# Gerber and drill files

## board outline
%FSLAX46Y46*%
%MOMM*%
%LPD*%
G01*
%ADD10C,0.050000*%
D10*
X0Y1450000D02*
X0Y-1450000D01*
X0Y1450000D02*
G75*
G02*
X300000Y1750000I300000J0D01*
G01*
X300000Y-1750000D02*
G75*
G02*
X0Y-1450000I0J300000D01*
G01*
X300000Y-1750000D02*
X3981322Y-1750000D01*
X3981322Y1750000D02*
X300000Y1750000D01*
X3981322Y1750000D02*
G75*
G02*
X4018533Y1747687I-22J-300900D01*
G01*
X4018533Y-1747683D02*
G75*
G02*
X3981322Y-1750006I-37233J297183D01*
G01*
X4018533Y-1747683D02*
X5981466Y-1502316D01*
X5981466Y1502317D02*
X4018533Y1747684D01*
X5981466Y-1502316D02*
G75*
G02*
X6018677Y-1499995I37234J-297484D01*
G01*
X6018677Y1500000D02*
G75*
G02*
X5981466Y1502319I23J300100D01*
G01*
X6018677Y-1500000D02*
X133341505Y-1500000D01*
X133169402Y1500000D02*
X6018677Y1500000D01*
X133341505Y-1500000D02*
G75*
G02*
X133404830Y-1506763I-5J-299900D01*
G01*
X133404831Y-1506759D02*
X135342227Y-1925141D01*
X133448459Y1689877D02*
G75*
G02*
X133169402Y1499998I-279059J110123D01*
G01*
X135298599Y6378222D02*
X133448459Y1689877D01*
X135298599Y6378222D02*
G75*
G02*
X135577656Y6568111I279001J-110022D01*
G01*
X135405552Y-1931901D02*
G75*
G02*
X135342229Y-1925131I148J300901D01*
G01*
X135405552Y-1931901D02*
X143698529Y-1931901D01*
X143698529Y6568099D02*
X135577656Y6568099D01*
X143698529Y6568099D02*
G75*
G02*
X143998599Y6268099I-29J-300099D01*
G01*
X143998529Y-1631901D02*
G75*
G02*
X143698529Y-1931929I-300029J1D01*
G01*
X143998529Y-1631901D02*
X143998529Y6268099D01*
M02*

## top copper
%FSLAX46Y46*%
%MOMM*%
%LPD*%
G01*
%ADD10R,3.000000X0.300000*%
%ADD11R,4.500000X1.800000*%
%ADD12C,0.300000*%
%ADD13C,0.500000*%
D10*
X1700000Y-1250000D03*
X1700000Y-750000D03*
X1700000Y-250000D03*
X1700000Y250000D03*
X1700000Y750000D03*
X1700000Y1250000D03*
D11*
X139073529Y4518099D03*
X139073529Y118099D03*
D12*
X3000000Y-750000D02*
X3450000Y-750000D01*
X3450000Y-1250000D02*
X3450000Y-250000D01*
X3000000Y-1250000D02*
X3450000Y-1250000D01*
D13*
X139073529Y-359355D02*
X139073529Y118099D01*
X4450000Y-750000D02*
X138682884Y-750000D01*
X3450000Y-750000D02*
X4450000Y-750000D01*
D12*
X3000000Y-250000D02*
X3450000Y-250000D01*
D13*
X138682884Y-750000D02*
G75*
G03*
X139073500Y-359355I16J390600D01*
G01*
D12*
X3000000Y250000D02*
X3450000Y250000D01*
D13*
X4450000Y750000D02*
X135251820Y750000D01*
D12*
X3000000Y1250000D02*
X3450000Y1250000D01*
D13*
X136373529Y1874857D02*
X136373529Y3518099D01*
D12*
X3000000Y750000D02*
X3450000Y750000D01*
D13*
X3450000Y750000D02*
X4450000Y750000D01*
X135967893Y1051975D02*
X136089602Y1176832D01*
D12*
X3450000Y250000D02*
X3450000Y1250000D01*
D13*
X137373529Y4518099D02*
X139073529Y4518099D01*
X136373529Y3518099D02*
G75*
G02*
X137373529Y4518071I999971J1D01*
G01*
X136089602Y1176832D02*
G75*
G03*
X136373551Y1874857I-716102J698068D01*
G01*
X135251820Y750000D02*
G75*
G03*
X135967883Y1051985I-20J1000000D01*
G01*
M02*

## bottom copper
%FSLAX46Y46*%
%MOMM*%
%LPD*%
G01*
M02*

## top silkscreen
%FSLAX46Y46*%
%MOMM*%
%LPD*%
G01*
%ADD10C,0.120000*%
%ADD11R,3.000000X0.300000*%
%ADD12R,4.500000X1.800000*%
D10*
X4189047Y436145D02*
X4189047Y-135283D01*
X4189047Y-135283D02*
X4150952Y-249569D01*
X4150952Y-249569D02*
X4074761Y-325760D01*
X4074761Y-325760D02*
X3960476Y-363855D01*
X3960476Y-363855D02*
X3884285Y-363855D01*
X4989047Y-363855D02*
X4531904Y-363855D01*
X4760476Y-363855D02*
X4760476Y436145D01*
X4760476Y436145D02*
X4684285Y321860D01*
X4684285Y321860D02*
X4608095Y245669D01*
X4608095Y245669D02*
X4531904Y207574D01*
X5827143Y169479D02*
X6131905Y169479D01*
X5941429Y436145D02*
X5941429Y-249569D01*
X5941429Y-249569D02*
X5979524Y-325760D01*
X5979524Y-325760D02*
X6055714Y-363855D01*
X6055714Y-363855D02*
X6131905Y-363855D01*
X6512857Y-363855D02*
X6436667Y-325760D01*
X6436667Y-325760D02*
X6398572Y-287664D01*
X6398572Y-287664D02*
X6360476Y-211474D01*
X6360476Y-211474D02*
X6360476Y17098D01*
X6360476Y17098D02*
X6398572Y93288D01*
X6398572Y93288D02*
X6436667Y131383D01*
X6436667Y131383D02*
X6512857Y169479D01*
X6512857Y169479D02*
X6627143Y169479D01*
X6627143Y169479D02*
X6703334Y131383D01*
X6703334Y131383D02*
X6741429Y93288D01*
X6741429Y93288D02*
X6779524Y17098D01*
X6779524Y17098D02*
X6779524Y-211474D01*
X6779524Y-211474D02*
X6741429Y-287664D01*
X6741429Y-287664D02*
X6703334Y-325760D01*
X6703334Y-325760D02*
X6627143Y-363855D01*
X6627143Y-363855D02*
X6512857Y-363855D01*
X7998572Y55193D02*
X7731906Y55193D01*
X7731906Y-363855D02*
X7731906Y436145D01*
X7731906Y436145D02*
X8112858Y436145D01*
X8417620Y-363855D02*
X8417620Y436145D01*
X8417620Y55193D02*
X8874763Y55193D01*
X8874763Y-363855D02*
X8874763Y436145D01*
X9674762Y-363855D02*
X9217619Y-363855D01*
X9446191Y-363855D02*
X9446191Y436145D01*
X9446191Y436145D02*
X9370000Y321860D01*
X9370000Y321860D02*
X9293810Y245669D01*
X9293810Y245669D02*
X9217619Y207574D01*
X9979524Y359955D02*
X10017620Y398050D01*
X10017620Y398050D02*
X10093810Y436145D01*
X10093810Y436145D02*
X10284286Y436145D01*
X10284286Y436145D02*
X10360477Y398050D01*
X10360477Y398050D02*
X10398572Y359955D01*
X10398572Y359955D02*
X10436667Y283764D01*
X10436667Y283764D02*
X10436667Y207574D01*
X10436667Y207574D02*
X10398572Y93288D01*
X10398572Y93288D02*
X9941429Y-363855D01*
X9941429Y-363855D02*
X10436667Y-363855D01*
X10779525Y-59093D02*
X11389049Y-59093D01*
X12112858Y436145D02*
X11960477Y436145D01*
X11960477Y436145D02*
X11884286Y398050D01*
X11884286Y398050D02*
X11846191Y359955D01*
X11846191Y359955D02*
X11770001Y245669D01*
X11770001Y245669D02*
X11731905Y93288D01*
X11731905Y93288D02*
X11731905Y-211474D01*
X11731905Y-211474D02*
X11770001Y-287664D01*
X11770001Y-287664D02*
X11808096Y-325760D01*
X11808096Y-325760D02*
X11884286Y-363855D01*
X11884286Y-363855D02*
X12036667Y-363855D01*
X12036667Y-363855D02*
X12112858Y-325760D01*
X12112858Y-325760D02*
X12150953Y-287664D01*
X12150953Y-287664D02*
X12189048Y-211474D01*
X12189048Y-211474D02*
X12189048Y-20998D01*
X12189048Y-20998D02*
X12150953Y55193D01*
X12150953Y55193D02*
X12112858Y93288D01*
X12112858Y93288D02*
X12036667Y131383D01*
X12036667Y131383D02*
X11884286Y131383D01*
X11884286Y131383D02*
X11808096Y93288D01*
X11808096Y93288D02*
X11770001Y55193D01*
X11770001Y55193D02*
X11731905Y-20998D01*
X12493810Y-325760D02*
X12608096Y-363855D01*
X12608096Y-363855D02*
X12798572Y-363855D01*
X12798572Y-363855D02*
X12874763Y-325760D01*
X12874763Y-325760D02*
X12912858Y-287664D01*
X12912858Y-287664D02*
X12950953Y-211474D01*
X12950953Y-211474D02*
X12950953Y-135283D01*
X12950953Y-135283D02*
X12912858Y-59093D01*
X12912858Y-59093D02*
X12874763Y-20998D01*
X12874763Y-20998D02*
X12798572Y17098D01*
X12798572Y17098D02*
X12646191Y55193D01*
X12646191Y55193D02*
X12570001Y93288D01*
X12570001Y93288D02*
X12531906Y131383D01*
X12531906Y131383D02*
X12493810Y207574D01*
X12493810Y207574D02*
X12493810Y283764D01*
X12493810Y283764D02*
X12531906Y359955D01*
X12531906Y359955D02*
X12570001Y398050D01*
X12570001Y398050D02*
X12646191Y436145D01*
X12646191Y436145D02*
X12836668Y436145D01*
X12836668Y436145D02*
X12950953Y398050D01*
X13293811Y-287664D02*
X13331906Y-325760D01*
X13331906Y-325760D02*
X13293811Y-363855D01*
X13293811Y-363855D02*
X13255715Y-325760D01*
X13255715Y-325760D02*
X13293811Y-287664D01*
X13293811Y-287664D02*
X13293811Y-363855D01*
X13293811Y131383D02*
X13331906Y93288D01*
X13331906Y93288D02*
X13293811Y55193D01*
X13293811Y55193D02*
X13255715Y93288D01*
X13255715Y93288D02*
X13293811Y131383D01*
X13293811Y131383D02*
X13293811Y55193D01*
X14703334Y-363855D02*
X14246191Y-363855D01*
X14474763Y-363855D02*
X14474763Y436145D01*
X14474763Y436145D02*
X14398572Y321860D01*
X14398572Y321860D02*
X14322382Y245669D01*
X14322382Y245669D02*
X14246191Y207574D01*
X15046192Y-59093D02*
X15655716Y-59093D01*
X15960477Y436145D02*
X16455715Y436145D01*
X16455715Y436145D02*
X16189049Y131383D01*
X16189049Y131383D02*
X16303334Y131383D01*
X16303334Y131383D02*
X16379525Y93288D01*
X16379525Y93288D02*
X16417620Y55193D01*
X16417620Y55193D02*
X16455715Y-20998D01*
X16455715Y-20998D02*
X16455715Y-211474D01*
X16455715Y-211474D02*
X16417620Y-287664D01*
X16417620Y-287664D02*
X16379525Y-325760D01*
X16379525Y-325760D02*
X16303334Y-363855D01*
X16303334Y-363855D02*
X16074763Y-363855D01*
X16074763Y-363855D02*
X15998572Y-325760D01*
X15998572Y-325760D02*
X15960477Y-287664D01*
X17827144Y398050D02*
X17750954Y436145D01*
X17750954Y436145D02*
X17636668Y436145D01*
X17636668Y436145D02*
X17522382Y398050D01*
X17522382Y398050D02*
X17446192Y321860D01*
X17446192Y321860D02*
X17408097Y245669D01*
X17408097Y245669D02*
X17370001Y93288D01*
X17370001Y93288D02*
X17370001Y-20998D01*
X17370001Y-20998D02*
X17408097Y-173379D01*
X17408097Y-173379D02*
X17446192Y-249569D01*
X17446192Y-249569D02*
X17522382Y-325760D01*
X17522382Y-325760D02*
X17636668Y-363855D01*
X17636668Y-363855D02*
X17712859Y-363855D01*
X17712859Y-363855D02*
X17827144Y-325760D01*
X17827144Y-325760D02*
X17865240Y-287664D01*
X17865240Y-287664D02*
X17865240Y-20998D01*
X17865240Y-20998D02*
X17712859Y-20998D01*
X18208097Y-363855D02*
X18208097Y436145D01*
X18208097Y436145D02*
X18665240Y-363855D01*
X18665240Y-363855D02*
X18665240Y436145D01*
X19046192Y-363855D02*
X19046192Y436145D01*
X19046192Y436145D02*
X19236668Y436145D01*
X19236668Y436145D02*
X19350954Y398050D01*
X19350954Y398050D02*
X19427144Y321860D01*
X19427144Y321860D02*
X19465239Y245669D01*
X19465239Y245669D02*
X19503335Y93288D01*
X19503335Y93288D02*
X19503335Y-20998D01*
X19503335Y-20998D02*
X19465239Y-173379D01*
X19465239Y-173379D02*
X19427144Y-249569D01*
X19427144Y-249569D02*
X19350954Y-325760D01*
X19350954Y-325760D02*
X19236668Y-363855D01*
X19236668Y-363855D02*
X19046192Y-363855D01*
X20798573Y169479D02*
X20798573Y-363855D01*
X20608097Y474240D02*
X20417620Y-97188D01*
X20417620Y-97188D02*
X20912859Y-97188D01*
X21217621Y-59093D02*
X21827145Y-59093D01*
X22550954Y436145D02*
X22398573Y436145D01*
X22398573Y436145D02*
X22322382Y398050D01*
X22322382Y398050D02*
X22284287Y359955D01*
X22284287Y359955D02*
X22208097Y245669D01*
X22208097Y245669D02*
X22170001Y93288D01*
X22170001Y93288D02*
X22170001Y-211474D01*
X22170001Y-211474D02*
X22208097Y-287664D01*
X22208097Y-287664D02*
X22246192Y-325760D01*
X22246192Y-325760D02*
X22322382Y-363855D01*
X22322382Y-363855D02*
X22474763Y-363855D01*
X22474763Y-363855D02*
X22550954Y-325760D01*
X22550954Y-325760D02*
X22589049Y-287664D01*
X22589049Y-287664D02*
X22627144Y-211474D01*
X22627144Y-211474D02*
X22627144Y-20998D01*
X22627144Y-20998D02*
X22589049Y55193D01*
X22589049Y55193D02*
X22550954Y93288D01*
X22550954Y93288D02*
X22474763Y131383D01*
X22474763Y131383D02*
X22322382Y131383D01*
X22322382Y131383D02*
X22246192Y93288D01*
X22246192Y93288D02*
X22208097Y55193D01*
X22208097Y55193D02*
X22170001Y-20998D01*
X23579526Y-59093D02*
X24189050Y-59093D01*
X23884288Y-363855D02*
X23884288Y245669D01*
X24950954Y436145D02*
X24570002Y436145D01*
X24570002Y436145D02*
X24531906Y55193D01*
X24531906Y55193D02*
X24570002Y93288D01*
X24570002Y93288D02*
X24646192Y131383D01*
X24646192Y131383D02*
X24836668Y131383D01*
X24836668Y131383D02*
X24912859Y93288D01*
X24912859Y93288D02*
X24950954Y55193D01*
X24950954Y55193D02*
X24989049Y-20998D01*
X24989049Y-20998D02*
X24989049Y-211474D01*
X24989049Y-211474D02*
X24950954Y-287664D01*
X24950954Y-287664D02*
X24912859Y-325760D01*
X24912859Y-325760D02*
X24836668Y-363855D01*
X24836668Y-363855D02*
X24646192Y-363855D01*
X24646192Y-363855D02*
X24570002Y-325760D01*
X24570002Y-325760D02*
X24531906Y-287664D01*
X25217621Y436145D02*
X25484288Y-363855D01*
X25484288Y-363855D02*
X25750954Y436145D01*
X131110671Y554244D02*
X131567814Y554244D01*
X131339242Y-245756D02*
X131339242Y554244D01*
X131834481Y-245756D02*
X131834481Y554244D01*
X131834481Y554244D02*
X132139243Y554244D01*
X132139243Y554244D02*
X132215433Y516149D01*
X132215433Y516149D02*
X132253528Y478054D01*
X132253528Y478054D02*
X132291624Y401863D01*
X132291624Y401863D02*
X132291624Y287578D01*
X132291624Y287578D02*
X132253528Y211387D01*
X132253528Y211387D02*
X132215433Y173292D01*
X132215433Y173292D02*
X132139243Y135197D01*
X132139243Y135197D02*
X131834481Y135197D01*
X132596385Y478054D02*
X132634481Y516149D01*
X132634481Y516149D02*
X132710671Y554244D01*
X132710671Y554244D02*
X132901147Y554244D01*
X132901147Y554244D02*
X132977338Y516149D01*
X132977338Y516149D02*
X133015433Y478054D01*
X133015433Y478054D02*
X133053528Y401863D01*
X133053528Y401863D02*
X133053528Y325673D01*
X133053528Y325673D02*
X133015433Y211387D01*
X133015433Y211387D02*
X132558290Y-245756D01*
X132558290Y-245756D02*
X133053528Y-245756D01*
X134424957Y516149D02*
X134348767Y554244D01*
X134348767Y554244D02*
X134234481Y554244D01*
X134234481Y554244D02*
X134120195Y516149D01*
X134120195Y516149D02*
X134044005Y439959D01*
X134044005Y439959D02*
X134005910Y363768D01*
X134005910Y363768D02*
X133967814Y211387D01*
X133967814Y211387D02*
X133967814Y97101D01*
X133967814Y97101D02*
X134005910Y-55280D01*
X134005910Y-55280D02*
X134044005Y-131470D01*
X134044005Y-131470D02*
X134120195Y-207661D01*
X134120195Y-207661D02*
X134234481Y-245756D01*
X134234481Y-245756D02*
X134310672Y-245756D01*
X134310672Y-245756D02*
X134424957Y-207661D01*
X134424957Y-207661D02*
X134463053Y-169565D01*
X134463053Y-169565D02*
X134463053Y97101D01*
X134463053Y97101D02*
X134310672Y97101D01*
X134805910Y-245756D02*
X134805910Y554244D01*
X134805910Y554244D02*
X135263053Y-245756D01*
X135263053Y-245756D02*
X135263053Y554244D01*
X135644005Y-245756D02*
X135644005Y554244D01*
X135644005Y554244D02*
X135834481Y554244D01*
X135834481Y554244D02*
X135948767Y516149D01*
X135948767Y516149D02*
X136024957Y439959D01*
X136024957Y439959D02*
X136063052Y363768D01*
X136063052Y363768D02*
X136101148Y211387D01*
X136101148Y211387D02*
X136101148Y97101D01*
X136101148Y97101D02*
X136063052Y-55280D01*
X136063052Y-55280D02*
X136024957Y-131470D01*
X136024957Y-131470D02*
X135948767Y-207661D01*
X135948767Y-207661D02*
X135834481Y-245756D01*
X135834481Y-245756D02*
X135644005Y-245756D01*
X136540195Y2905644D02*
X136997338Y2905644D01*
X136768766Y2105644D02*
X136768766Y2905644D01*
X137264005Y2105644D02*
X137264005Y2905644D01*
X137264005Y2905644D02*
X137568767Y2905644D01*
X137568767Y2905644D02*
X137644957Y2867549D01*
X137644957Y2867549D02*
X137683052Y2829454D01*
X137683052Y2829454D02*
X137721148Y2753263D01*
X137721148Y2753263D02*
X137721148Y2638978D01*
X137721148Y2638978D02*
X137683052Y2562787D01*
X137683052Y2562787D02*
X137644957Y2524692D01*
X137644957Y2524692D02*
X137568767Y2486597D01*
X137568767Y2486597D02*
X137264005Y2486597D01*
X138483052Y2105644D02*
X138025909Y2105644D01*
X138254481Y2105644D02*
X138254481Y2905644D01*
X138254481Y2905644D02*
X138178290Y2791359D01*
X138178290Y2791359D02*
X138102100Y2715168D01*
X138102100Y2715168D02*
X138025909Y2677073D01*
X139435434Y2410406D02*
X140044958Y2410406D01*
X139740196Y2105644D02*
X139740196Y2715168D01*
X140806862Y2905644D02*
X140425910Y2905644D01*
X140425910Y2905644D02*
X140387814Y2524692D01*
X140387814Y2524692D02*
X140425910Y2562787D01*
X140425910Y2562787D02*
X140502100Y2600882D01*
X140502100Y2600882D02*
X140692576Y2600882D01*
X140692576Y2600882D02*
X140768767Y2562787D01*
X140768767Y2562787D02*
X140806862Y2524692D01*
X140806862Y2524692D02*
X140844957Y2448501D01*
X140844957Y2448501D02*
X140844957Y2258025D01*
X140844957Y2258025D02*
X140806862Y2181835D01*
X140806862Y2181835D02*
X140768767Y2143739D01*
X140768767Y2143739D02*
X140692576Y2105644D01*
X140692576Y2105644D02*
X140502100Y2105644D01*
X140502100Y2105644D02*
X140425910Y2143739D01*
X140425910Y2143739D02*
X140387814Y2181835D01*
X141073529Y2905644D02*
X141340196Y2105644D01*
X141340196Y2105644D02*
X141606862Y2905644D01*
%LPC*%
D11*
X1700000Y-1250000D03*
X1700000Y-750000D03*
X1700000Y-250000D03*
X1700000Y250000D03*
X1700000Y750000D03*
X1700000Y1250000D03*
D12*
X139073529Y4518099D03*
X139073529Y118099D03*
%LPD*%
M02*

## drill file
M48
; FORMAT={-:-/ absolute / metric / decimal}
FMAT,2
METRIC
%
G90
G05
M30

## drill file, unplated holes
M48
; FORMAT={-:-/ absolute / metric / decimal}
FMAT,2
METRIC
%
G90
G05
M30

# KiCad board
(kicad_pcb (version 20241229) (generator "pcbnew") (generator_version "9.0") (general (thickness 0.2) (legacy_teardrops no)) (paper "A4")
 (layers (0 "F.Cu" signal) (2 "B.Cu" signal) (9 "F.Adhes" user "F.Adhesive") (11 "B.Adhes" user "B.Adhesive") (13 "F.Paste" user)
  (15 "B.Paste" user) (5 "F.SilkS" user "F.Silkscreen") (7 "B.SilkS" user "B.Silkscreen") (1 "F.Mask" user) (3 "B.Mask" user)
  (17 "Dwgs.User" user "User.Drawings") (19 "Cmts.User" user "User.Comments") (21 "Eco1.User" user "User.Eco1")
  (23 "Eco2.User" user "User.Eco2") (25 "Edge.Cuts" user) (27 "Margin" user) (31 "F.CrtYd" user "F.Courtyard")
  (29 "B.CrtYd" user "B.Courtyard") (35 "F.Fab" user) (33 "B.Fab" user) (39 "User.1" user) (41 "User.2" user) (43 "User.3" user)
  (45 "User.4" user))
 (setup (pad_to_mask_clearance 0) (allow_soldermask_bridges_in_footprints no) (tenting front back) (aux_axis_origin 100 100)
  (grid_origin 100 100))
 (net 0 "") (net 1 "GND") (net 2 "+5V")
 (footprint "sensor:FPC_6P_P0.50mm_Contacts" (layer "F.Cu") (at 101.7 100)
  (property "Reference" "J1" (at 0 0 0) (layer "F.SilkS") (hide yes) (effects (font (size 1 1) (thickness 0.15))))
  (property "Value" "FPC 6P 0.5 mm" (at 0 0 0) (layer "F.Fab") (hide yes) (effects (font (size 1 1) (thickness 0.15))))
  (pad "1" smd rect (at 0 1.25) (size 3 0.3) (layers "F.Cu" "F.Mask") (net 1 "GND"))
  (pad "2" smd rect (at 0 0.75) (size 3 0.3) (layers "F.Cu" "F.Mask") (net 1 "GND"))
  (pad "3" smd rect (at 0 0.25) (size 3 0.3) (layers "F.Cu" "F.Mask") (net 1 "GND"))
  (pad "4" smd rect (at 0 -0.25) (size 3 0.3) (layers "F.Cu" "F.Mask") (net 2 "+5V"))
  (pad "5" smd rect (at 0 -0.75) (size 3 0.3) (layers "F.Cu" "F.Mask") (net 2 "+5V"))
  (pad "6" smd rect (at 0 -1.25) (size 3 0.3) (layers "F.Cu" "F.Mask") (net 2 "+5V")))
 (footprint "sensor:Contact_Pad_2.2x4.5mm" (layer "F.Cu") (at 239.073529 95.481901)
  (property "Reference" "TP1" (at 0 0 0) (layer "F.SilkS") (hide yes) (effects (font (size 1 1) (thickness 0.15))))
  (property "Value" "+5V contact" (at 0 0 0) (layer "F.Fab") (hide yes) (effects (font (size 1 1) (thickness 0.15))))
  (pad "1" smd rect (at 0 0) (size 4.5 1.8) (layers "F.Cu" "F.Mask") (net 2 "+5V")))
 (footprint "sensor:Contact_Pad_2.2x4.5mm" (layer "F.Cu") (at 239.073529 99.881901)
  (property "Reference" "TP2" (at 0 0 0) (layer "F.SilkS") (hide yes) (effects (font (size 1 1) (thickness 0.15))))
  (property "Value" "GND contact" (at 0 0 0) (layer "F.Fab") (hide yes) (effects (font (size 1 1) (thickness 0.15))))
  (pad "1" smd rect (at 0 0) (size 4.5 1.8) (layers "F.Cu" "F.Mask") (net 1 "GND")))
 (gr_line (start 100 98.55) (end 100 101.45) (stroke (width 0.05) (type default)) (layer "Edge.Cuts"))
 (gr_arc (start 100 98.55) (mid 100.087868 98.337868) (end 100.3 98.25) (stroke (width 0.05) (type default)) (layer "Edge.Cuts"))
 (gr_arc (start 100.3 101.75) (mid 100.087868 101.662132) (end 100 101.45) (stroke (width 0.05) (type default)) (layer "Edge.Cuts"))
 (gr_line (start 100.3 101.75) (end 103.981322 101.75) (stroke (width 0.05) (type default)) (layer "Edge.Cuts"))
 (gr_line (start 103.981322 98.25) (end 100.3 98.25) (stroke (width 0.05) (type default)) (layer "Edge.Cuts"))
 (gr_arc (start 103.981322 98.25) (mid 103.999963 98.250581) (end 104.018533 98.252316) (stroke (width 0.05) (type default))
  (layer "Edge.Cuts"))
 (gr_arc (start 104.018533 101.747683) (mid 103.999964 101.749421) (end 103.981322 101.75) (stroke (width 0.05) (type default))
  (layer "Edge.Cuts"))
 (gr_line (start 104.018533 101.747683) (end 105.981466 101.502316) (stroke (width 0.05) (type default)) (layer "Edge.Cuts"))
 (gr_line (start 105.981466 98.497683) (end 104.018533 98.252316) (stroke (width 0.05) (type default)) (layer "Edge.Cuts"))
 (gr_arc (start 105.981466 101.502316) (mid 106.000036 101.500579) (end 106.018677 101.5) (stroke (width 0.05) (type default))
  (layer "Edge.Cuts"))
 (gr_arc (start 106.018677 98.5) (mid 106.000036 98.49942) (end 105.981466 98.497683) (stroke (width 0.05) (type default))
  (layer "Edge.Cuts"))
 (gr_line (start 106.018677 101.5) (end 233.341505 101.5) (stroke (width 0.05) (type default)) (layer "Edge.Cuts"))
 (gr_line (start 233.169402 98.5) (end 106.018677 98.5) (stroke (width 0.05) (type default)) (layer "Edge.Cuts"))
 (gr_arc (start 233.341505 101.5) (mid 233.373348 101.501694) (end 233.404831 101.506759) (stroke (width 0.05) (type default))
  (layer "Edge.Cuts"))
 (gr_line (start 233.404831 101.506759) (end 235.342227 101.925141) (stroke (width 0.05) (type default)) (layer "Edge.Cuts"))
 (gr_arc (start 233.448459 98.310123) (mid 233.338167 98.448029) (end 233.169402 98.5) (stroke (width 0.05) (type default))
  (layer "Edge.Cuts"))
 (gr_line (start 235.298599 93.621778) (end 233.448459 98.310123) (stroke (width 0.05) (type default)) (layer "Edge.Cuts"))
 (gr_arc (start 235.298599 93.621778) (mid 235.408887 93.483855) (end 235.577656 93.431901) (stroke (width 0.05) (type default))
  (layer "Edge.Cuts"))
 (gr_arc (start 235.405552 101.931901) (mid 235.37371 101.930201) (end 235.342227 101.925141) (stroke (width 0.05) (type default))
  (layer "Edge.Cuts"))
 (gr_line (start 235.405552 101.931901) (end 243.698529 101.931901) (stroke (width 0.05) (type default)) (layer "Edge.Cuts"))
 (gr_line (start 243.698529 93.431901) (end 235.577656 93.431901) (stroke (width 0.05) (type default)) (layer "Edge.Cuts"))
 (gr_arc (start 243.698529 93.431901) (mid 243.910642 93.519779) (end 243.998529 93.731901) (stroke (width 0.05) (type default))
  (layer "Edge.Cuts"))
 (gr_arc (start 243.998529 101.631901) (mid 243.910662 101.844043) (end 243.698529 101.931901) (stroke (width 0.05) (type default))
  (layer "Edge.Cuts"))
 (gr_line (start 243.998529 101.631901) (end 243.998529 93.731901) (stroke (width 0.05) (type default)) (layer "Edge.Cuts"))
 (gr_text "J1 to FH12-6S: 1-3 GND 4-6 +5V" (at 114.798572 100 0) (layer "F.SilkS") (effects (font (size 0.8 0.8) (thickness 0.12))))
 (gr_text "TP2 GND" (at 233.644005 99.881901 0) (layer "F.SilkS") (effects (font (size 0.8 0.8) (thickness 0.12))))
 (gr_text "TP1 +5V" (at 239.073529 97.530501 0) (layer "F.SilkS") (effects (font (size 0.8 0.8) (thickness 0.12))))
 (segment (start 103 100.75) (end 103.45 100.75) (width 0.3) (layer "F.Cu") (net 1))
 (segment (start 103.45 101.25) (end 103.45 100.25) (width 0.3) (layer "F.Cu") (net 1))
 (segment (start 103 101.25) (end 103.45 101.25) (width 0.3) (layer "F.Cu") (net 1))
 (segment (start 239.073529 100.359355) (end 239.073529 99.881901) (width 0.5) (layer "F.Cu") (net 1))
 (segment (start 104.45 100.75) (end 238.682884 100.75) (width 0.5) (layer "F.Cu") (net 1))
 (segment (start 103.45 100.75) (end 104.45 100.75) (width 0.5) (layer "F.Cu") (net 1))
 (segment (start 103 100.25) (end 103.45 100.25) (width 0.3) (layer "F.Cu") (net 1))
 (arc (start 238.682884 100.75) (mid 238.959111 100.635582) (end 239.073529 100.359355) (width 0.5) (layer "F.Cu") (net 1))
 (segment (start 103 99.75) (end 103.45 99.75) (width 0.3) (layer "F.Cu") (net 2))
 (segment (start 104.45 99.25) (end 235.25182 99.25) (width 0.5) (layer "F.Cu") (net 2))
 (segment (start 103 98.75) (end 103.45 98.75) (width 0.3) (layer "F.Cu") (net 2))
 (segment (start 236.373529 98.125143) (end 236.373529 96.481901) (width 0.5) (layer "F.Cu") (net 2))
 (segment (start 103 99.25) (end 103.45 99.25) (width 0.3) (layer "F.Cu") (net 2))
 (segment (start 103.45 99.25) (end 104.45 99.25) (width 0.5) (layer "F.Cu") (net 2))
 (segment (start 235.967893 98.948025) (end 236.089602 98.823168) (width 0.5) (layer "F.Cu") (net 2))
 (segment (start 103.45 99.75) (end 103.45 98.75) (width 0.3) (layer "F.Cu") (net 2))
 (segment (start 237.373529 95.481901) (end 239.073529 95.481901) (width 0.5) (layer "F.Cu") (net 2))
 (arc (start 236.373529 96.481901) (mid 236.666422 95.774794) (end 237.373529 95.481901) (width 0.5) (layer "F.Cu") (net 2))
 (arc (start 236.089602 98.823168) (mid 236.299832 98.501924) (end 236.373529 98.125143) (width 0.5) (layer "F.Cu") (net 2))
 (arc (start 235.25182 99.25) (mid 235.64039 99.171418) (end 235.967893 98.948025) (width 0.5) (layer "F.Cu") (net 2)))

